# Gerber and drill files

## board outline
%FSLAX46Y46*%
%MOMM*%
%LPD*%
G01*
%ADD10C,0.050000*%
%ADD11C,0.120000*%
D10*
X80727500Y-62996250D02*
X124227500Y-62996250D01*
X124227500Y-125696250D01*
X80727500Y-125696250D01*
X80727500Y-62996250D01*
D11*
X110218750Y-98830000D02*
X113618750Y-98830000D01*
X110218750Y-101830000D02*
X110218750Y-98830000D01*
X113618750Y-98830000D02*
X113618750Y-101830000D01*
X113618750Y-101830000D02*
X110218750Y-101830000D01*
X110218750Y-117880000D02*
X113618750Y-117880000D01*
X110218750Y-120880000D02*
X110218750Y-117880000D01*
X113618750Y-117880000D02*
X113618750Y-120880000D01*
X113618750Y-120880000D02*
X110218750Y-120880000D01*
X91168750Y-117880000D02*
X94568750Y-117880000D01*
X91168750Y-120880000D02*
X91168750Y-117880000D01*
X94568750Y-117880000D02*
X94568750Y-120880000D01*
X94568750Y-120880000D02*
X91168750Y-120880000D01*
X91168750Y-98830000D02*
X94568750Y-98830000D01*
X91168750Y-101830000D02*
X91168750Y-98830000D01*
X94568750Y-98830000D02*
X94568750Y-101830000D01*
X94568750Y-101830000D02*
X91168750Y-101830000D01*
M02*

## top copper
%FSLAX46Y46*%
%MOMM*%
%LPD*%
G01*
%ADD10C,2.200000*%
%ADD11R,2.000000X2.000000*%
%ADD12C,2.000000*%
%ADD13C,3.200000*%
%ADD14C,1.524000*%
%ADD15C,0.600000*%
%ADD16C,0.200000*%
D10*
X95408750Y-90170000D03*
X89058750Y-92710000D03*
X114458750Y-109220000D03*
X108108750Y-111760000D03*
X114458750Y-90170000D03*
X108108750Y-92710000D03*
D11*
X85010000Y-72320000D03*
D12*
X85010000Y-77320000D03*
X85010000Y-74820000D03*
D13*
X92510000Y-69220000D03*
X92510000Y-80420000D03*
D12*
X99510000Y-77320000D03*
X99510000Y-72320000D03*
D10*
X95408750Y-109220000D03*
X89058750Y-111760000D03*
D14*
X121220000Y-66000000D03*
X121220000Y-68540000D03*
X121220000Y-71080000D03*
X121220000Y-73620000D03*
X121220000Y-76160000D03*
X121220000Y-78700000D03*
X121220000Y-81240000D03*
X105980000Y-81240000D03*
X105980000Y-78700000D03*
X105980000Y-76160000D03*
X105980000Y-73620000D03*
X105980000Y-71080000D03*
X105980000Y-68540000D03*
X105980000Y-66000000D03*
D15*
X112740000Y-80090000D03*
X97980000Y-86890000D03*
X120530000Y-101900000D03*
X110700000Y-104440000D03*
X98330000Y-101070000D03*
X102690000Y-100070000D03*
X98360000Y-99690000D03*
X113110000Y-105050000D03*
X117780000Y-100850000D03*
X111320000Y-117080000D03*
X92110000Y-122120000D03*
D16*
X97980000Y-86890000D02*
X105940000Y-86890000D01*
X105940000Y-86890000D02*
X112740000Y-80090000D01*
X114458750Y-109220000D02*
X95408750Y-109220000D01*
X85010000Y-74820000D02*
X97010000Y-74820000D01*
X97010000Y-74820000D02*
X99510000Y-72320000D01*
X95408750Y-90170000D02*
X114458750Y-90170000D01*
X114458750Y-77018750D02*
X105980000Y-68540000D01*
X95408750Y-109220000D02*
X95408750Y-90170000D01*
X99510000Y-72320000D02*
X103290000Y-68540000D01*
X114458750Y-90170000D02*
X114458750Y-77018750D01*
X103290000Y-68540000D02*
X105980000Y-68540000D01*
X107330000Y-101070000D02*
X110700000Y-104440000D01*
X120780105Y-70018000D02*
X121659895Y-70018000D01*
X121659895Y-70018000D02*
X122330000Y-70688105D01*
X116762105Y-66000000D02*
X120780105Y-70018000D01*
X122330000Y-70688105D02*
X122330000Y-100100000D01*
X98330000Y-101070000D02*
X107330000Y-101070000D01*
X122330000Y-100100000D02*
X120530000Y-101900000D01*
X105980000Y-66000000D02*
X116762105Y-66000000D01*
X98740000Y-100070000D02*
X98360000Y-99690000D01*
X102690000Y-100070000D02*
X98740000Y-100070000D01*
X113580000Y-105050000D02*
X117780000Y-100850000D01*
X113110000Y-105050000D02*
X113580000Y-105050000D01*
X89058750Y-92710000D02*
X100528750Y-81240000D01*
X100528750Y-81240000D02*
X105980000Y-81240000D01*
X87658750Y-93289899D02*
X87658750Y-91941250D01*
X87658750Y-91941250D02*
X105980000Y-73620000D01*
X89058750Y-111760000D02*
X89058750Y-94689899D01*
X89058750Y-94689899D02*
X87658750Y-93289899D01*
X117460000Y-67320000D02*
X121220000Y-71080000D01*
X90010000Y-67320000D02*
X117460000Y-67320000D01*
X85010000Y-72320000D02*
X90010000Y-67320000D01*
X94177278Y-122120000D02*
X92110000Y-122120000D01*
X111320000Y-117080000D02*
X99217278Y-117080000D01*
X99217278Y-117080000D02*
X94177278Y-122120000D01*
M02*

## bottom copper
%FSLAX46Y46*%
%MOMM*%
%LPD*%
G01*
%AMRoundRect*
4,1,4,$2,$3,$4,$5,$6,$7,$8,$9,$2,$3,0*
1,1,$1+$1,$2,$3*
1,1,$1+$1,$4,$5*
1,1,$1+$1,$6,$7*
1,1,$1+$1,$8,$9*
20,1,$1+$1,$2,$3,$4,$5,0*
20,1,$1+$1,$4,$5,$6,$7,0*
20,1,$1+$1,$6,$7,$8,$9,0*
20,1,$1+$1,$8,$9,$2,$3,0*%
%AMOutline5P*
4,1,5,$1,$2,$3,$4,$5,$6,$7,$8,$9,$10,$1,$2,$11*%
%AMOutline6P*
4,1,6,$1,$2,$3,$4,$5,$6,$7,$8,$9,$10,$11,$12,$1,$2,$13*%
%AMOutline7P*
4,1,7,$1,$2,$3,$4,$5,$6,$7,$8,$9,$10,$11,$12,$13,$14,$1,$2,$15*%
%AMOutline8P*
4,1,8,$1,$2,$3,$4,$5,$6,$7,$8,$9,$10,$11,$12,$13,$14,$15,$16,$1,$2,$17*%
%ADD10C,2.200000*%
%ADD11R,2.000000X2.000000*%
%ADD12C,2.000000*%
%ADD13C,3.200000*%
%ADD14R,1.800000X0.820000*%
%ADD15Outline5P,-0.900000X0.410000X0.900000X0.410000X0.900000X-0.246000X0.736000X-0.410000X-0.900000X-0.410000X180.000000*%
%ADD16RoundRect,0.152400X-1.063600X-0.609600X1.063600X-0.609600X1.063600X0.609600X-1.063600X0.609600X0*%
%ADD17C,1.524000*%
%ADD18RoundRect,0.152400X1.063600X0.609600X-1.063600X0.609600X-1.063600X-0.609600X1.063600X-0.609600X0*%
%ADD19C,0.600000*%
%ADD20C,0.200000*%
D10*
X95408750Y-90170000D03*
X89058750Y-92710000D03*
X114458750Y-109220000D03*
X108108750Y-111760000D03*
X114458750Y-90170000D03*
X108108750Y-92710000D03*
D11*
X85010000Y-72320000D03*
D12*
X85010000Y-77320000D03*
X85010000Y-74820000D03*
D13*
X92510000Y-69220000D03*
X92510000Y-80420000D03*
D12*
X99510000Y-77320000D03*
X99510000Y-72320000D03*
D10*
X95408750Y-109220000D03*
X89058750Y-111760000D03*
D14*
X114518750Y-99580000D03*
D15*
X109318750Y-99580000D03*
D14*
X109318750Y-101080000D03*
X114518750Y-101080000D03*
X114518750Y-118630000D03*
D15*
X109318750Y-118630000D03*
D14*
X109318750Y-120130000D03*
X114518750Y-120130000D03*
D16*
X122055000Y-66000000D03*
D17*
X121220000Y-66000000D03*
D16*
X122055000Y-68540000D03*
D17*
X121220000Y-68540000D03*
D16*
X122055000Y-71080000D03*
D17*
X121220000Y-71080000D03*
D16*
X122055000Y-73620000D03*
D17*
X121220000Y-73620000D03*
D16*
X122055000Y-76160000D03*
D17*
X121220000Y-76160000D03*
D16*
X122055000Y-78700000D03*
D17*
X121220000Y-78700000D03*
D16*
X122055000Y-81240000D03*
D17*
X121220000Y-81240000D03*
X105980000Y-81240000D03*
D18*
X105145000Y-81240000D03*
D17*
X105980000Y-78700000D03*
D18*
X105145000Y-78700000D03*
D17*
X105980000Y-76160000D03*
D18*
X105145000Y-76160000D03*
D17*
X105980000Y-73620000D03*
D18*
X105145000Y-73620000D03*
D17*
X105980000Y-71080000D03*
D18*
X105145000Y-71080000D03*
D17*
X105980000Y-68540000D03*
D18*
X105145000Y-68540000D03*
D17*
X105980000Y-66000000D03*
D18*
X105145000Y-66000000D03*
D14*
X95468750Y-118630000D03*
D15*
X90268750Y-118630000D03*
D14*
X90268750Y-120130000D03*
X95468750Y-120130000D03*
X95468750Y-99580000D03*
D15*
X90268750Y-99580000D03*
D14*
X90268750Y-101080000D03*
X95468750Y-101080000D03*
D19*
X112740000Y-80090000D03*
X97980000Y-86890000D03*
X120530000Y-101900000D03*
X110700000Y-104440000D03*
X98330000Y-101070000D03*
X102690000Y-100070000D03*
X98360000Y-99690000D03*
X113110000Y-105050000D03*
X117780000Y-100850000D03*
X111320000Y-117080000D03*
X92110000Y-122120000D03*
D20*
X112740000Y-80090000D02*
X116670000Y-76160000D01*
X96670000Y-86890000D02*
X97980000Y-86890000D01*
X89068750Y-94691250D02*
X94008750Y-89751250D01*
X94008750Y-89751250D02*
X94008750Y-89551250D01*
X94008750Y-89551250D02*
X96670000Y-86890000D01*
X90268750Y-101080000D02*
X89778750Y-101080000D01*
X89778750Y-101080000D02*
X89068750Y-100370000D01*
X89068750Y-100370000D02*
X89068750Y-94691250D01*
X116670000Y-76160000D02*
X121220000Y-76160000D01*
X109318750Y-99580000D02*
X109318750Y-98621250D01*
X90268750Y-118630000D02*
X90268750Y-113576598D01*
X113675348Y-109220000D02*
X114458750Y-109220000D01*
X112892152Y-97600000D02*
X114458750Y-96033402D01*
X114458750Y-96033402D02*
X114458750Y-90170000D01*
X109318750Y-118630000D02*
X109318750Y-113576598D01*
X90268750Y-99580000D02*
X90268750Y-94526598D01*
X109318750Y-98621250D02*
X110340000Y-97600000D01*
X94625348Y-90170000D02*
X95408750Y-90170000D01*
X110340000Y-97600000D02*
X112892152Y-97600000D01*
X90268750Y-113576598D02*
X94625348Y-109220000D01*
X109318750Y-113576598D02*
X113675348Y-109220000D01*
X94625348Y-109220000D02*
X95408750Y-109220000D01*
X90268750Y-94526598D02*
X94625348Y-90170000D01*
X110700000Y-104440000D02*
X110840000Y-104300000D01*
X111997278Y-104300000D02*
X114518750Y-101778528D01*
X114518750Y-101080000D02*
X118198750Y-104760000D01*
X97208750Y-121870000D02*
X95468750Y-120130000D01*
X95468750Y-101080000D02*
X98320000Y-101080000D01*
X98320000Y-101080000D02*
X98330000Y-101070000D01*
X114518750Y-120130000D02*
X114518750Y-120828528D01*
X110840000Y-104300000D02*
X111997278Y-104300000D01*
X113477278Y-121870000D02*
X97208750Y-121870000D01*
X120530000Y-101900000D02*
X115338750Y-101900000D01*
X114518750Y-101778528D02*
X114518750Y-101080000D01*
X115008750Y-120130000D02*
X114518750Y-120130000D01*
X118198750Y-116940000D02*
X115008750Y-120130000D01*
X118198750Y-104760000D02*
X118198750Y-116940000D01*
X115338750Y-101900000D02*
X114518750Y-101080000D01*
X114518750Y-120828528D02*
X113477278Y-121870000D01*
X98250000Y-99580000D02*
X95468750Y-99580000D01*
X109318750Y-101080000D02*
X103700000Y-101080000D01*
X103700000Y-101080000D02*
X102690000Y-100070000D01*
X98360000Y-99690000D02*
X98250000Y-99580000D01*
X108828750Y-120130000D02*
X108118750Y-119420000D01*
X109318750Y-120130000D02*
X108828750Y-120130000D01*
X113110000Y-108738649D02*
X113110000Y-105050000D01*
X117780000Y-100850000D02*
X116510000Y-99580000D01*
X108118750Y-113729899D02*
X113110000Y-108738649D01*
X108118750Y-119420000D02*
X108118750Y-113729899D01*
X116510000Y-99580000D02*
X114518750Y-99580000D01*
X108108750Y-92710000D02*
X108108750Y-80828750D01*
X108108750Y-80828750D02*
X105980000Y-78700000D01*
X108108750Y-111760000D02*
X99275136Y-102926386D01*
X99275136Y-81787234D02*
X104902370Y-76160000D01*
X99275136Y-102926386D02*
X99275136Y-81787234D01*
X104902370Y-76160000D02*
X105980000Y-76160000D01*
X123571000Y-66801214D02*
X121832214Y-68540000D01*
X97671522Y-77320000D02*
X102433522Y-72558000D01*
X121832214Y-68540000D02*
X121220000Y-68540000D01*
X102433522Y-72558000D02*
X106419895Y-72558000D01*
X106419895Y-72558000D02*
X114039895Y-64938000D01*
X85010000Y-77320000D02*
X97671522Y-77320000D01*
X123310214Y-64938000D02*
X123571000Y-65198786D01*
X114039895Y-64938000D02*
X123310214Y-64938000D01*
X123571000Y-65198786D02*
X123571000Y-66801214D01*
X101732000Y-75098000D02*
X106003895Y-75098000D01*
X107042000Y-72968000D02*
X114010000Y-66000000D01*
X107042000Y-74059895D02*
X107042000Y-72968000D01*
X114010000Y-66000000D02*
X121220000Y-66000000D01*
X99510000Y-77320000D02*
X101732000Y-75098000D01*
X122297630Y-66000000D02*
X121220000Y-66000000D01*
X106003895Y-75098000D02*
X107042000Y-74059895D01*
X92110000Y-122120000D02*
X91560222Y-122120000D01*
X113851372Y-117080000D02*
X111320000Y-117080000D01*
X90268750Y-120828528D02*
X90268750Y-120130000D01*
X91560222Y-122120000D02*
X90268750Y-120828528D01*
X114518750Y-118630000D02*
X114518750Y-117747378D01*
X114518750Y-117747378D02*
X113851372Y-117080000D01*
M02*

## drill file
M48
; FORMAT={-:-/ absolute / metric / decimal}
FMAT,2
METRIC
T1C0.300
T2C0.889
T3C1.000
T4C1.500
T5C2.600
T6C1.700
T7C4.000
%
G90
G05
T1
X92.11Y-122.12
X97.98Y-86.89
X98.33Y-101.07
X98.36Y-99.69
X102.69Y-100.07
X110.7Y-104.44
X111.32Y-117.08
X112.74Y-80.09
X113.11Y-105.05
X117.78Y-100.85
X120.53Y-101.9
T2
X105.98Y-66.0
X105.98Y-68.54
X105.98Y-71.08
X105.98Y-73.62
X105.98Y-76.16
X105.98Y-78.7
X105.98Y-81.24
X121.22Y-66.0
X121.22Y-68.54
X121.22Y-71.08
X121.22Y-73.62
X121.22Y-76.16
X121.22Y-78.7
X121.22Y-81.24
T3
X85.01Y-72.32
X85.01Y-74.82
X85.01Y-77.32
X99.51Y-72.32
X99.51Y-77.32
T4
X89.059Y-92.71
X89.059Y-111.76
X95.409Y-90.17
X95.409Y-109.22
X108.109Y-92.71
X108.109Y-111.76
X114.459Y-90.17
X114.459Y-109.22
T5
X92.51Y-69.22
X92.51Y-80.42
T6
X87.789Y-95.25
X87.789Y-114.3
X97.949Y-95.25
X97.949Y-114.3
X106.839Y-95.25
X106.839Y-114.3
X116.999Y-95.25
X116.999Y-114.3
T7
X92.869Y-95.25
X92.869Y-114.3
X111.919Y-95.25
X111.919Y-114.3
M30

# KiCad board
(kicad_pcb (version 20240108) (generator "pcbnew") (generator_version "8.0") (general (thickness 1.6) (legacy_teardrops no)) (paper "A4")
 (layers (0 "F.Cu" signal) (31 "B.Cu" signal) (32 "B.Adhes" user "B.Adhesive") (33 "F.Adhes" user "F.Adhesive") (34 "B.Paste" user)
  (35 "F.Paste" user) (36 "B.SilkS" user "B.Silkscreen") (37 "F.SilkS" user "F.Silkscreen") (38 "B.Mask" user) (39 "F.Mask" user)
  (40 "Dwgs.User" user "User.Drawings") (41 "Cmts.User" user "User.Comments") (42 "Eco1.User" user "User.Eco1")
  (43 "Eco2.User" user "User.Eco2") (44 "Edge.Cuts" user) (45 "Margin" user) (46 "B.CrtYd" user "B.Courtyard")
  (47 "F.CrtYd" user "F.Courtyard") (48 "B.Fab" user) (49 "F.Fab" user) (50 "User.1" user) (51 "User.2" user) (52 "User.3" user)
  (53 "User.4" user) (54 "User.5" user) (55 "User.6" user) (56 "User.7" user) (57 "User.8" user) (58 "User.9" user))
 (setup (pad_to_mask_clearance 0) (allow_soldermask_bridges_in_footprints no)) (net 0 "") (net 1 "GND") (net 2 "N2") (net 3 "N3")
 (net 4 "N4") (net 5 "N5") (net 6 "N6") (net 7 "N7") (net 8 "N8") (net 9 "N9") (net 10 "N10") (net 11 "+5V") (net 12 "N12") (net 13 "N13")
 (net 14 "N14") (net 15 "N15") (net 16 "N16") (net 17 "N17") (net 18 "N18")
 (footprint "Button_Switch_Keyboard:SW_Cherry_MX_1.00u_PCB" (layer "F.Cu") (at 95.40875 90.17)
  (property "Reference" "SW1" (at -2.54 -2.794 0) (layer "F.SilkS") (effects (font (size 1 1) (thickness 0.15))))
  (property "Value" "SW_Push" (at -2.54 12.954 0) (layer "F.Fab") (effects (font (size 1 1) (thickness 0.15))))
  (pad "" np_thru_hole circle (at -7.62 5.08) (size 1.7 1.7) (drill 1.7) (layers "*.Cu" "*.Mask"))
  (pad "" np_thru_hole circle (at -2.54 5.08) (size 4 4) (drill 4) (layers "*.Cu" "*.Mask"))
  (pad "" np_thru_hole circle (at 2.54 5.08) (size 1.7 1.7) (drill 1.7) (layers "*.Cu" "*.Mask"))
  (pad "1" thru_hole circle (at 0 0) (size 2.2 2.2) (drill 1.5) (layers "*.Cu" "*.Mask") (remove_unused_layers no) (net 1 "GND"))
  (pad "2" thru_hole circle (at -6.35 2.54) (size 2.2 2.2) (drill 1.5) (layers "*.Cu" "*.Mask") (remove_unused_layers no) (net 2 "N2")))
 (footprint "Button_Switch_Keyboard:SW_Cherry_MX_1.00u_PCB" (layer "F.Cu") (at 114.45875 109.22)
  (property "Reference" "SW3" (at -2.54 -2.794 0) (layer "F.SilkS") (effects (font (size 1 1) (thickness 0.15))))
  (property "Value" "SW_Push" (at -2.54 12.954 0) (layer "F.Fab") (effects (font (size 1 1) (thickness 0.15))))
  (pad "" np_thru_hole circle (at -7.62 5.08) (size 1.7 1.7) (drill 1.7) (layers "*.Cu" "*.Mask"))
  (pad "" np_thru_hole circle (at -2.54 5.08) (size 4 4) (drill 4) (layers "*.Cu" "*.Mask"))
  (pad "" np_thru_hole circle (at 2.54 5.08) (size 1.7 1.7) (drill 1.7) (layers "*.Cu" "*.Mask"))
  (pad "1" thru_hole circle (at 0 0) (size 2.2 2.2) (drill 1.5) (layers "*.Cu" "*.Mask") (remove_unused_layers no) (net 1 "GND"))
  (pad "2" thru_hole circle (at -6.35 2.54) (size 2.2 2.2) (drill 1.5) (layers "*.Cu" "*.Mask") (remove_unused_layers no) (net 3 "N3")))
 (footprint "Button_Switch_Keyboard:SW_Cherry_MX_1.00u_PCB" (layer "F.Cu") (at 114.45875 90.17)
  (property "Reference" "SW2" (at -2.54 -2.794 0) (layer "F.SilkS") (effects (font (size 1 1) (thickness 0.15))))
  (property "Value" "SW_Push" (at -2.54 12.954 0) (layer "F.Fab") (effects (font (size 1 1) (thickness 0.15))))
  (pad "" np_thru_hole circle (at -7.62 5.08) (size 1.7 1.7) (drill 1.7) (layers "*.Cu" "*.Mask"))
  (pad "" np_thru_hole circle (at -2.54 5.08) (size 4 4) (drill 4) (layers "*.Cu" "*.Mask"))
  (pad "" np_thru_hole circle (at 2.54 5.08) (size 1.7 1.7) (drill 1.7) (layers "*.Cu" "*.Mask"))
  (pad "1" thru_hole circle (at 0 0) (size 2.2 2.2) (drill 1.5) (layers "*.Cu" "*.Mask") (remove_unused_layers no) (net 1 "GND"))
  (pad "2" thru_hole circle (at -6.35 2.54) (size 2.2 2.2) (drill 1.5) (layers "*.Cu" "*.Mask") (remove_unused_layers no) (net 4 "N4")))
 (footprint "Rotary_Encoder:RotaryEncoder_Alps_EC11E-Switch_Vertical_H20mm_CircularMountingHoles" (layer "F.Cu") (at 85.01 72.32)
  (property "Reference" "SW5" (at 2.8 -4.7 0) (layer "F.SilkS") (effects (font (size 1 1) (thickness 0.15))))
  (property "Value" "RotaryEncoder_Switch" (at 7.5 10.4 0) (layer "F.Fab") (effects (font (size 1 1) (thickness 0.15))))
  (pad "A" thru_hole rect (at 0 0) (size 2 2) (drill 1) (layers "*.Cu" "*.Mask") (remove_unused_layers no) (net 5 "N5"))
  (pad "B" thru_hole circle (at 0 5) (size 2 2) (drill 1) (layers "*.Cu" "*.Mask") (remove_unused_layers no) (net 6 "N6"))
  (pad "C" thru_hole circle (at 0 2.5) (size 2 2) (drill 1) (layers "*.Cu" "*.Mask") (remove_unused_layers no) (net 1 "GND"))
  (pad "MP" thru_hole circle (at 7.5 -3.1) (size 3.2 3.2) (drill 2.6) (layers "*.Cu" "*.Mask") (remove_unused_layers no))
  (pad "MP" thru_hole circle (at 7.5 8.1) (size 3.2 3.2) (drill 2.6) (layers "*.Cu" "*.Mask") (remove_unused_layers no))
  (pad "S1" thru_hole circle (at 14.5 5) (size 2 2) (drill 1) (layers "*.Cu" "*.Mask") (remove_unused_layers no) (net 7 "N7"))
  (pad "S2" thru_hole circle (at 14.5 0) (size 2 2) (drill 1) (layers "*.Cu" "*.Mask") (remove_unused_layers no) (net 1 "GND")))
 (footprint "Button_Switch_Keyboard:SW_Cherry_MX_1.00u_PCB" (layer "F.Cu") (at 95.40875 109.22)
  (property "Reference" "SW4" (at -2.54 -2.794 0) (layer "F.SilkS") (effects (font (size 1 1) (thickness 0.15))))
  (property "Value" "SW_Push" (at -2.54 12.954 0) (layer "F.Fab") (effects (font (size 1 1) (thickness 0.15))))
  (pad "" np_thru_hole circle (at -7.62 5.08) (size 1.7 1.7) (drill 1.7) (layers "*.Cu" "*.Mask"))
  (pad "" np_thru_hole circle (at -2.54 5.08) (size 4 4) (drill 4) (layers "*.Cu" "*.Mask"))
  (pad "" np_thru_hole circle (at 2.54 5.08) (size 1.7 1.7) (drill 1.7) (layers "*.Cu" "*.Mask"))
  (pad "1" thru_hole circle (at 0 0) (size 2.2 2.2) (drill 1.5) (layers "*.Cu" "*.Mask") (remove_unused_layers no) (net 1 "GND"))
  (pad "2" thru_hole circle (at -6.35 2.54) (size 2.2 2.2) (drill 1.5) (layers "*.Cu" "*.Mask") (remove_unused_layers no) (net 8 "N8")))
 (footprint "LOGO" (layer "B.Cu") (at 101.67 98.78 180)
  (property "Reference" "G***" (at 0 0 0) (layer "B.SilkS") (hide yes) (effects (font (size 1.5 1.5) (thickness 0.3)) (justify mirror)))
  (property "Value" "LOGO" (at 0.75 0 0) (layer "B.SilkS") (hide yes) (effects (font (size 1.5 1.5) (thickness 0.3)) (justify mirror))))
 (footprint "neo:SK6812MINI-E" (layer "B.Cu") (at 111.91875 100.33 180)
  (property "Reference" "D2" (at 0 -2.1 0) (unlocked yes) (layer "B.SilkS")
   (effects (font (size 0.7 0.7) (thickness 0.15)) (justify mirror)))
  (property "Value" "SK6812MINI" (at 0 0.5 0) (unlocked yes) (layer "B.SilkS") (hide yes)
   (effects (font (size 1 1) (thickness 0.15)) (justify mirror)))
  (fp_line (start 1.7 1.5) (end -1.7 1.5) (stroke (width 0.12) (type solid)) (layer "Edge.Cuts"))
  (fp_line (start 1.7 -1.5) (end 1.7 1.5) (stroke (width 0.12) (type solid)) (layer "Edge.Cuts"))
  (fp_line (start -1.7 1.5) (end -1.7 -1.5) (stroke (width 0.12) (type solid)) (layer "Edge.Cuts"))
  (fp_line (start -1.7 -1.5) (end 1.7 -1.5) (stroke (width 0.12) (type solid)) (layer "Edge.Cuts"))
  (pad "1" smd rect (at -2.6 0.75 180) (size 1.8 0.82) (layers "B.Cu" "B.Paste" "B.Mask") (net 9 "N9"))
  (pad "2" smd roundrect (at 2.6 0.75 180) (size 1.8 0.82) (layers "B.Cu" "B.Paste" "B.Mask") (roundrect_rratio 0) (chamfer_ratio 0.2)
   (chamfer bottom_right) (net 1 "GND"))
  (pad "3" smd rect (at 2.6 -0.75 180) (size 1.8 0.82) (layers "B.Cu" "B.Paste" "B.Mask") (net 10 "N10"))
  (pad "4" smd rect (at -2.6 -0.75 180) (size 1.8 0.82) (layers "B.Cu" "B.Paste" "B.Mask") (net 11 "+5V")))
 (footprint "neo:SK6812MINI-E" (layer "B.Cu") (at 111.91875 119.38 180)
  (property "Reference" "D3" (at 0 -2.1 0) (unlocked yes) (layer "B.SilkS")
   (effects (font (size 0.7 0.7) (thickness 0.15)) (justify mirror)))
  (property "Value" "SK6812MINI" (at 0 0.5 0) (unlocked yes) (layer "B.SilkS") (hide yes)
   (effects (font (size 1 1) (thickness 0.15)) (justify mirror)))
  (fp_line (start 1.7 1.5) (end -1.7 1.5) (stroke (width 0.12) (type solid)) (layer "Edge.Cuts"))
  (fp_line (start 1.7 -1.5) (end 1.7 1.5) (stroke (width 0.12) (type solid)) (layer "Edge.Cuts"))
  (fp_line (start -1.7 1.5) (end -1.7 -1.5) (stroke (width 0.12) (type solid)) (layer "Edge.Cuts"))
  (fp_line (start -1.7 -1.5) (end 1.7 -1.5) (stroke (width 0.12) (type solid)) (layer "Edge.Cuts"))
  (pad "1" smd rect (at -2.6 0.75 180) (size 1.8 0.82) (layers "B.Cu" "B.Paste" "B.Mask") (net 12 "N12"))
  (pad "2" smd roundrect (at 2.6 0.75 180) (size 1.8 0.82) (layers "B.Cu" "B.Paste" "B.Mask") (roundrect_rratio 0) (chamfer_ratio 0.2)
   (chamfer bottom_right) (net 1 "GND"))
  (pad "3" smd rect (at 2.6 -0.75 180) (size 1.8 0.82) (layers "B.Cu" "B.Paste" "B.Mask") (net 9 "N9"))
  (pad "4" smd rect (at -2.6 -0.75 180) (size 1.8 0.82) (layers "B.Cu" "B.Paste" "B.Mask") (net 11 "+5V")))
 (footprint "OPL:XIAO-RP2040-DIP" (layer "B.Cu") (at 113.6 73.62 180)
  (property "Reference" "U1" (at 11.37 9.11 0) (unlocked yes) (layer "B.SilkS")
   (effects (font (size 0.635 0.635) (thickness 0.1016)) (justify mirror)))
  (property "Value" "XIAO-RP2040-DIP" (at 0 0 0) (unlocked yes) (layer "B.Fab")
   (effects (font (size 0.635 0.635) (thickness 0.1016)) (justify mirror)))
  (pad "1" smd roundrect (at -8.455 7.62) (size 2.432 1.524) (layers "B.Cu" "B.Mask") (roundrect_rratio 0.1) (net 7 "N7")
   (thermal_bridge_angle 45))
  (pad "1" thru_hole circle (at -7.62 7.62) (size 1.524 1.524) (drill 0.889) (layers "*.Cu" "*.Mask") (remove_unused_layers no) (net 7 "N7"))
  (pad "2" smd roundrect (at -8.455 5.08) (size 2.432 1.524) (layers "B.Cu" "B.Mask") (roundrect_rratio 0.1) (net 6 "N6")
   (thermal_bridge_angle 45))
  (pad "2" thru_hole circle (at -7.62 5.08) (size 1.524 1.524) (drill 0.889) (layers "*.Cu" "*.Mask") (remove_unused_layers no) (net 6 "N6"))
  (pad "3" smd roundrect (at -8.455 2.54) (size 2.432 1.524) (layers "B.Cu" "B.Mask") (roundrect_rratio 0.1) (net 5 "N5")
   (thermal_bridge_angle 45))
  (pad "3" thru_hole circle (at -7.62 2.54) (size 1.524 1.524) (drill 0.889) (layers "*.Cu" "*.Mask") (remove_unused_layers no) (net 5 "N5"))
  (pad "4" smd roundrect (at -8.455 0) (size 2.432 1.524) (layers "B.Cu" "B.Mask") (roundrect_rratio 0.1) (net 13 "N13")
   (thermal_bridge_angle 45))
  (pad "4" thru_hole circle (at -7.62 0) (size 1.524 1.524) (drill 0.889) (layers "*.Cu" "*.Mask") (remove_unused_layers no) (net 13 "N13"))
  (pad "5" smd roundrect (at -8.455 -2.54) (size 2.432 1.524) (layers "B.Cu" "B.Mask") (roundrect_rratio 0.1) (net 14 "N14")
   (thermal_bridge_angle 45))
  (pad "5" thru_hole circle (at -7.62 -2.54) (size 1.524 1.524) (drill 0.889) (layers "*.Cu" "*.Mask") (remove_unused_layers no)
   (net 14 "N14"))
  (pad "6" smd roundrect (at -8.455 -5.08) (size 2.432 1.524) (layers "B.Cu" "B.Mask") (roundrect_rratio 0.1) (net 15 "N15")
   (thermal_bridge_angle 45))
  (pad "6" thru_hole circle (at -7.62 -5.08) (size 1.524 1.524) (drill 0.889) (layers "*.Cu" "*.Mask") (remove_unused_layers no)
   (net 15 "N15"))
  (pad "7" smd roundrect (at -8.455 -7.62) (size 2.432 1.524) (layers "B.Cu" "B.Mask") (roundrect_rratio 0.1) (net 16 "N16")
   (thermal_bridge_angle 45))
  (pad "7" thru_hole circle (at -7.62 -7.62) (size 1.524 1.524) (drill 0.889) (layers "*.Cu" "*.Mask") (remove_unused_layers no)
   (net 16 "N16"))
  (pad "8" thru_hole circle (at 7.62 -7.62 180) (size 1.524 1.524) (drill 0.889) (layers "*.Cu" "*.Mask") (remove_unused_layers no)
   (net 2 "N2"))
  (pad "8" smd roundrect (at 8.455 -7.62 180) (size 2.432 1.524) (layers "B.Cu" "B.Mask") (roundrect_rratio 0.1) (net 2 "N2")
   (thermal_bridge_angle 45))
  (pad "9" thru_hole circle (at 7.62 -5.08 180) (size 1.524 1.524) (drill 0.889) (layers "*.Cu" "*.Mask") (remove_unused_layers no)
   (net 4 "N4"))
  (pad "9" smd roundrect (at 8.455 -5.08 180) (size 2.432 1.524) (layers "B.Cu" "B.Mask") (roundrect_rratio 0.1) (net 4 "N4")
   (thermal_bridge_angle 45))
  (pad "10" thru_hole circle (at 7.62 -2.54 180) (size 1.524 1.524) (drill 0.889) (layers "*.Cu" "*.Mask") (remove_unused_layers no)
   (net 3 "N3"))
  (pad "10" smd roundrect (at 8.455 -2.54 180) (size 2.432 1.524) (layers "B.Cu" "B.Mask") (roundrect_rratio 0.1) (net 3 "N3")
   (thermal_bridge_angle 45))
  (pad "11" thru_hole circle (at 7.62 0 180) (size 1.524 1.524) (drill 0.889) (layers "*.Cu" "*.Mask") (remove_unused_layers no)
   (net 8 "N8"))
  (pad "11" smd roundrect (at 8.455 0 180) (size 2.432 1.524) (layers "B.Cu" "B.Mask") (roundrect_rratio 0.1) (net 8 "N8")
   (thermal_bridge_angle 45))
  (pad "12" thru_hole circle (at 7.62 2.54 180) (size 1.524 1.524) (drill 0.889) (layers "*.Cu" "*.Mask") (remove_unused_layers no)
   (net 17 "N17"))
  (pad "12" smd roundrect (at 8.455 2.54 180) (size 2.432 1.524) (layers "B.Cu" "B.Mask") (roundrect_rratio 0.1) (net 17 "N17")
   (thermal_bridge_angle 45))
  (pad "13" thru_hole circle (at 7.62 5.08 180) (size 1.524 1.524) (drill 0.889) (layers "*.Cu" "*.Mask") (remove_unused_layers no)
   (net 1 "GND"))
  (pad "13" smd roundrect (at 8.455 5.08 180) (size 2.432 1.524) (layers "B.Cu" "B.Mask") (roundrect_rratio 0.1) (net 1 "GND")
   (thermal_bridge_angle 45))
  (pad "14" thru_hole circle (at 7.62 7.62 180) (size 1.524 1.524) (drill 0.889) (layers "*.Cu" "*.Mask") (remove_unused_layers no)
   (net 11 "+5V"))
  (pad "14" smd roundrect (at 8.455 7.62 180) (size 2.432 1.524) (layers "B.Cu" "B.Mask") (roundrect_rratio 0.1) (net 11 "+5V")
   (thermal_bridge_angle 45)))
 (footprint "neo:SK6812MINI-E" (layer "B.Cu") (at 92.86875 119.38 180)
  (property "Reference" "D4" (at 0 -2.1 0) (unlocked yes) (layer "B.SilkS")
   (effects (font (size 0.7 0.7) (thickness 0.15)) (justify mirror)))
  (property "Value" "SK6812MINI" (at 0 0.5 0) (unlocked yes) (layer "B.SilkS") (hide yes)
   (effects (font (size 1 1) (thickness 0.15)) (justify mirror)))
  (fp_line (start 1.7 1.5) (end -1.7 1.5) (stroke (width 0.12) (type solid)) (layer "Edge.Cuts"))
  (fp_line (start 1.7 -1.5) (end 1.7 1.5) (stroke (width 0.12) (type solid)) (layer "Edge.Cuts"))
  (fp_line (start -1.7 1.5) (end -1.7 -1.5) (stroke (width 0.12) (type solid)) (layer "Edge.Cuts"))
  (fp_line (start -1.7 -1.5) (end 1.7 -1.5) (stroke (width 0.12) (type solid)) (layer "Edge.Cuts"))
  (pad "1" smd rect (at -2.6 0.75 180) (size 1.8 0.82) (layers "B.Cu" "B.Paste" "B.Mask") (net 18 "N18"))
  (pad "2" smd roundrect (at 2.6 0.75 180) (size 1.8 0.82) (layers "B.Cu" "B.Paste" "B.Mask") (roundrect_rratio 0) (chamfer_ratio 0.2)
   (chamfer bottom_right) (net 1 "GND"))
  (pad "3" smd rect (at 2.6 -0.75 180) (size 1.8 0.82) (layers "B.Cu" "B.Paste" "B.Mask") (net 12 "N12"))
  (pad "4" smd rect (at -2.6 -0.75 180) (size 1.8 0.82) (layers "B.Cu" "B.Paste" "B.Mask") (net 11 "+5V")))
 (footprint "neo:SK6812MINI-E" (layer "B.Cu") (at 92.86875 100.33 180)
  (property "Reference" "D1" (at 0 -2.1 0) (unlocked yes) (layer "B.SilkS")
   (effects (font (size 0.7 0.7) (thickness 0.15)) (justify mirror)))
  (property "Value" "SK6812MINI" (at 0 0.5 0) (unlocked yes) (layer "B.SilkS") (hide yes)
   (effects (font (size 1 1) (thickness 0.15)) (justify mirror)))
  (fp_line (start 1.7 1.5) (end -1.7 1.5) (stroke (width 0.12) (type solid)) (layer "Edge.Cuts"))
  (fp_line (start 1.7 -1.5) (end 1.7 1.5) (stroke (width 0.12) (type solid)) (layer "Edge.Cuts"))
  (fp_line (start -1.7 1.5) (end -1.7 -1.5) (stroke (width 0.12) (type solid)) (layer "Edge.Cuts"))
  (fp_line (start -1.7 -1.5) (end 1.7 -1.5) (stroke (width 0.12) (type solid)) (layer "Edge.Cuts"))
  (pad "1" smd rect (at -2.6 0.75 180) (size 1.8 0.82) (layers "B.Cu" "B.Paste" "B.Mask") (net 10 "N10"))
  (pad "2" smd roundrect (at 2.6 0.75 180) (size 1.8 0.82) (layers "B.Cu" "B.Paste" "B.Mask") (roundrect_rratio 0) (chamfer_ratio 0.2)
   (chamfer bottom_right) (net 1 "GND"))
  (pad "3" smd rect (at 2.6 -0.75 180) (size 1.8 0.82) (layers "B.Cu" "B.Paste" "B.Mask") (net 14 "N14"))
  (pad "4" smd rect (at -2.6 -0.75 180) (size 1.8 0.82) (layers "B.Cu" "B.Paste" "B.Mask") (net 11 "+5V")))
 (gr_rect (start 80.7275 62.99625) (end 124.2275 125.69625) (stroke (width 0.05) (type default)) (fill none) (layer "Edge.Cuts"))
 (segment (start 97.98 86.89) (end 105.94 86.89) (width 0.2) (layer "F.Cu") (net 14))
 (segment (start 105.94 86.89) (end 112.74 80.09) (width 0.2) (layer "F.Cu") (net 14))
 (via (at 112.74 80.09) (size 0.6) (drill 0.3) (layers "F.Cu" "B.Cu") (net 14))
 (via (at 97.98 86.89) (size 0.6) (drill 0.3) (layers "F.Cu" "B.Cu") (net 14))
 (segment (start 112.74 80.09) (end 116.67 76.16) (width 0.2) (layer "B.Cu") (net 14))
 (segment (start 96.67 86.89) (end 97.98 86.89) (width 0.2) (layer "B.Cu") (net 14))
 (segment (start 89.06875 94.69125) (end 94.00875 89.75125) (width 0.2) (layer "B.Cu") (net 14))
 (segment (start 94.00875 89.75125) (end 94.00875 89.55125) (width 0.2) (layer "B.Cu") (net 14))
 (segment (start 94.00875 89.55125) (end 96.67 86.89) (width 0.2) (layer "B.Cu") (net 14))
 (segment (start 90.26875 101.08) (end 89.77875 101.08) (width 0.2) (layer "B.Cu") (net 14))
 (segment (start 89.77875 101.08) (end 89.06875 100.37) (width 0.2) (layer "B.Cu") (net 14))
 (segment (start 89.06875 100.37) (end 89.06875 94.69125) (width 0.2) (layer "B.Cu") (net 14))
 (segment (start 116.67 76.16) (end 121.22 76.16) (width 0.2) (layer "B.Cu") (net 14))
 (segment (start 114.45875 109.22) (end 95.40875 109.22) (width 0.2) (layer "F.Cu") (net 1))
 (segment (start 85.01 74.82) (end 97.01 74.82) (width 0.2) (layer "F.Cu") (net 1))
 (segment (start 97.01 74.82) (end 99.51 72.32) (width 0.2) (layer "F.Cu") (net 1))
 (segment (start 95.40875 90.17) (end 114.45875 90.17) (width 0.2) (layer "F.Cu") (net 1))
 (segment (start 114.45875 77.01875) (end 105.98 68.54) (width 0.2) (layer "F.Cu") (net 1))
 (segment (start 95.40875 109.22) (end 95.40875 90.17) (width 0.2) (layer "F.Cu") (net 1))
 (segment (start 99.51 72.32) (end 103.29 68.54) (width 0.2) (layer "F.Cu") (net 1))
 (segment (start 114.45875 90.17) (end 114.45875 77.01875) (width 0.2) (layer "F.Cu") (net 1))
 (segment (start 103.29 68.54) (end 105.98 68.54) (width 0.2) (layer "F.Cu") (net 1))
 (segment (start 109.31875 99.58) (end 109.31875 98.62125) (width 0.2) (layer "B.Cu") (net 1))
 (segment (start 90.26875 118.63) (end 90.26875 113.576598) (width 0.2) (layer "B.Cu") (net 1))
 (segment (start 113.675348 109.22) (end 114.45875 109.22) (width 0.2) (layer "B.Cu") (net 1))
 (segment (start 112.892152 97.6) (end 114.45875 96.033402) (width 0.2) (layer "B.Cu") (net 1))
 (segment (start 114.45875 96.033402) (end 114.45875 90.17) (width 0.2) (layer "B.Cu") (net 1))
 (segment (start 109.31875 118.63) (end 109.31875 113.576598) (width 0.2) (layer "B.Cu") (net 1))
 (segment (start 90.26875 99.58) (end 90.26875 94.526598) (width 0.2) (layer "B.Cu") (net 1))
 (segment (start 109.31875 98.62125) (end 110.34 97.6) (width 0.2) (layer "B.Cu") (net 1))
 (segment (start 94.625348 90.17) (end 95.40875 90.17) (width 0.2) (layer "B.Cu") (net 1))
 (segment (start 110.34 97.6) (end 112.892152 97.6) (width 0.2) (layer "B.Cu") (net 1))
 (segment (start 90.26875 113.576598) (end 94.625348 109.22) (width 0.2) (layer "B.Cu") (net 1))
 (segment (start 109.31875 113.576598) (end 113.675348 109.22) (width 0.2) (layer "B.Cu") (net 1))
 (segment (start 94.625348 109.22) (end 95.40875 109.22) (width 0.2) (layer "B.Cu") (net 1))
 (segment (start 90.26875 94.526598) (end 94.625348 90.17) (width 0.2) (layer "B.Cu") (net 1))
 (segment (start 107.33 101.07) (end 110.7 104.44) (width 0.2) (layer "F.Cu") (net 11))
 (segment (start 120.780105 70.018) (end 121.659895 70.018) (width 0.2) (layer "F.Cu") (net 11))
 (segment (start 121.659895 70.018) (end 122.33 70.688105) (width 0.2) (layer "F.Cu") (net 11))
 (segment (start 116.762105 66) (end 120.780105 70.018) (width 0.2) (layer "F.Cu") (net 11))
 (segment (start 122.33 70.688105) (end 122.33 100.1) (width 0.2) (layer "F.Cu") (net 11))
 (segment (start 98.33 101.07) (end 107.33 101.07) (width 0.2) (layer "F.Cu") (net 11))
 (segment (start 122.33 100.1) (end 120.53 101.9) (width 0.2) (layer "F.Cu") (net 11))
 (segment (start 105.98 66) (end 116.762105 66) (width 0.2) (layer "F.Cu") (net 11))
 (via (at 120.53 101.9) (size 0.6) (drill 0.3) (layers "F.Cu" "B.Cu") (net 11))
 (via (at 110.7 104.44) (size 0.6) (drill 0.3) (layers "F.Cu" "B.Cu") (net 11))
 (via (at 98.33 101.07) (size 0.6) (drill 0.3) (layers "F.Cu" "B.Cu") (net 11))
 (segment (start 110.7 104.44) (end 110.84 104.3) (width 0.2) (layer "B.Cu") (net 11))
 (segment (start 111.997278 104.3) (end 114.51875 101.778528) (width 0.2) (layer "B.Cu") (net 11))
 (segment (start 114.51875 101.08) (end 118.19875 104.76) (width 0.2) (layer "B.Cu") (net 11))
 (segment (start 97.20875 121.87) (end 95.46875 120.13) (width 0.2) (layer "B.Cu") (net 11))
 (segment (start 95.46875 101.08) (end 98.32 101.08) (width 0.2) (layer "B.Cu") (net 11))
 (segment (start 98.32 101.08) (end 98.33 101.07) (width 0.2) (layer "B.Cu") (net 11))
 (segment (start 114.51875 120.13) (end 114.51875 120.828528) (width 0.2) (layer "B.Cu") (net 11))
 (segment (start 110.84 104.3) (end 111.997278 104.3) (width 0.2) (layer "B.Cu") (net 11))
 (segment (start 113.477278 121.87) (end 97.20875 121.87) (width 0.2) (layer "B.Cu") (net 11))
 (segment (start 120.53 101.9) (end 115.33875 101.9) (width 0.2) (layer "B.Cu") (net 11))
 (segment (start 114.51875 101.778528) (end 114.51875 101.08) (width 0.2) (layer "B.Cu") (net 11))
 (segment (start 115.00875 120.13) (end 114.51875 120.13) (width 0.2) (layer "B.Cu") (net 11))
 (segment (start 118.19875 116.94) (end 115.00875 120.13) (width 0.2) (layer "B.Cu") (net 11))
 (segment (start 118.19875 104.76) (end 118.19875 116.94) (width 0.2) (layer "B.Cu") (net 11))
 (segment (start 115.33875 101.9) (end 114.51875 101.08) (width 0.2) (layer "B.Cu") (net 11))
 (segment (start 114.51875 120.828528) (end 113.477278 121.87) (width 0.2) (layer "B.Cu") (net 11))
 (segment (start 98.74 100.07) (end 98.36 99.69) (width 0.2) (layer "F.Cu") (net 10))
 (segment (start 102.69 100.07) (end 98.74 100.07) (width 0.2) (layer "F.Cu") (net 10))
 (via (at 102.69 100.07) (size 0.6) (drill 0.3) (layers "F.Cu" "B.Cu") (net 10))
 (via (at 98.36 99.69) (size 0.6) (drill 0.3) (layers "F.Cu" "B.Cu") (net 10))
 (segment (start 98.25 99.58) (end 95.46875 99.58) (width 0.2) (layer "B.Cu") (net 10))
 (segment (start 109.31875 101.08) (end 103.7 101.08) (width 0.2) (layer "B.Cu") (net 10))
 (segment (start 103.7 101.08) (end 102.69 100.07) (width 0.2) (layer "B.Cu") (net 10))
 (segment (start 98.36 99.69) (end 98.25 99.58) (width 0.2) (layer "B.Cu") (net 10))
 (segment (start 113.58 105.05) (end 117.78 100.85) (width 0.2) (layer "F.Cu") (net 9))
 (segment (start 113.11 105.05) (end 113.58 105.05) (width 0.2) (layer "F.Cu") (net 9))
 (via (at 113.11 105.05) (size 0.6) (drill 0.3) (layers "F.Cu" "B.Cu") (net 9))
 (via (at 117.78 100.85) (size 0.6) (drill 0.3) (layers "F.Cu" "B.Cu") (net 9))
 (segment (start 108.82875 120.13) (end 108.11875 119.42) (width 0.2) (layer "B.Cu") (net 9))
 (segment (start 109.31875 120.13) (end 108.82875 120.13) (width 0.2) (layer "B.Cu") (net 9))
 (segment (start 113.11 108.738649) (end 113.11 105.05) (width 0.2) (layer "B.Cu") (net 9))
 (segment (start 117.78 100.85) (end 116.51 99.58) (width 0.2) (layer "B.Cu") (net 9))
 (segment (start 108.11875 113.729899) (end 113.11 108.738649) (width 0.2) (layer "B.Cu") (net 9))
 (segment (start 108.11875 119.42) (end 108.11875 113.729899) (width 0.2) (layer "B.Cu") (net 9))
 (segment (start 116.51 99.58) (end 114.51875 99.58) (width 0.2) (layer "B.Cu") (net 9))
 (segment (start 89.05875 92.71) (end 100.52875 81.24) (width 0.2) (layer "F.Cu") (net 2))
 (segment (start 100.52875 81.24) (end 105.98 81.24) (width 0.2) (layer "F.Cu") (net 2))
 (segment (start 108.10875 92.71) (end 108.10875 80.82875) (width 0.2) (layer "B.Cu") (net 4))
 (segment (start 108.10875 80.82875) (end 105.98 78.7) (width 0.2) (layer "B.Cu") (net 4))
 (segment (start 108.10875 111.76) (end 99.275136 102.926386) (width 0.2) (layer "B.Cu") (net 3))
 (segment (start 99.275136 81.787234) (end 104.90237 76.16) (width 0.2) (layer "B.Cu") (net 3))
 (segment (start 99.275136 102.926386) (end 99.275136 81.787234) (width 0.2) (layer "B.Cu") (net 3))
 (segment (start 104.90237 76.16) (end 105.98 76.16) (width 0.2) (layer "B.Cu") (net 3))
 (segment (start 87.65875 93.289899) (end 87.65875 91.94125) (width 0.2) (layer "F.Cu") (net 8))
 (segment (start 87.65875 91.94125) (end 105.98 73.62) (width 0.2) (layer "F.Cu") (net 8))
 (segment (start 89.05875 111.76) (end 89.05875 94.689899) (width 0.2) (layer "F.Cu") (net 8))
 (segment (start 89.05875 94.689899) (end 87.65875 93.289899) (width 0.2) (layer "F.Cu") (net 8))
 (segment (start 123.571 66.801214) (end 121.832214 68.54) (width 0.2) (layer "B.Cu") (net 6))
 (segment (start 97.671522 77.32) (end 102.433522 72.558) (width 0.2) (layer "B.Cu") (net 6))
 (segment (start 121.832214 68.54) (end 121.22 68.54) (width 0.2) (layer "B.Cu") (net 6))
 (segment (start 102.433522 72.558) (end 106.419895 72.558) (width 0.2) (layer "B.Cu") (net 6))
 (segment (start 106.419895 72.558) (end 114.039895 64.938) (width 0.2) (layer "B.Cu") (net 6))
 (segment (start 85.01 77.32) (end 97.671522 77.32) (width 0.2) (layer "B.Cu") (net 6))
 (segment (start 123.310214 64.938) (end 123.571 65.198786) (width 0.2) (layer "B.Cu") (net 6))
 (segment (start 114.039895 64.938) (end 123.310214 64.938) (width 0.2) (layer "B.Cu") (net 6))
 (segment (start 123.571 65.198786) (end 123.571 66.801214) (width 0.2) (layer "B.Cu") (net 6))
 (segment (start 117.46 67.32) (end 121.22 71.08) (width 0.2) (layer "F.Cu") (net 5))
 (segment (start 90.01 67.32) (end 117.46 67.32) (width 0.2) (layer "F.Cu") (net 5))
 (segment (start 85.01 72.32) (end 90.01 67.32) (width 0.2) (layer "F.Cu") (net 5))
 (segment (start 101.732 75.098) (end 106.003895 75.098) (width 0.2) (layer "B.Cu") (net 7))
 (segment (start 107.042 72.968) (end 114.01 66) (width 0.2) (layer "B.Cu") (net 7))
 (segment (start 107.042 74.059895) (end 107.042 72.968) (width 0.2) (layer "B.Cu") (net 7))
 (segment (start 114.01 66) (end 121.22 66) (width 0.2) (layer "B.Cu") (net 7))
 (segment (start 99.51 77.32) (end 101.732 75.098) (width 0.2) (layer "B.Cu") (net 7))
 (segment (start 122.29763 66) (end 121.22 66) (width 0.2) (layer "B.Cu") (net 7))
 (segment (start 106.003895 75.098) (end 107.042 74.059895) (width 0.2) (layer "B.Cu") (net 7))
 (segment (start 94.177278 122.12) (end 92.11 122.12) (width 0.2) (layer "F.Cu") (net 12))
 (segment (start 111.32 117.08) (end 99.217278 117.08) (width 0.2) (layer "F.Cu") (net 12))
 (segment (start 99.217278 117.08) (end 94.177278 122.12) (width 0.2) (layer "F.Cu") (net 12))
 (via (at 111.32 117.08) (size 0.6) (drill 0.3) (layers "F.Cu" "B.Cu") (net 12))
 (via (at 92.11 122.12) (size 0.6) (drill 0.3) (layers "F.Cu" "B.Cu") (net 12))
 (segment (start 92.11 122.12) (end 91.560222 122.12) (width 0.2) (layer "B.Cu") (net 12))
 (segment (start 113.851372 117.08) (end 111.32 117.08) (width 0.2) (layer "B.Cu") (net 12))
 (segment (start 90.26875 120.828528) (end 90.26875 120.13) (width 0.2) (layer "B.Cu") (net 12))
 (segment (start 91.560222 122.12) (end 90.26875 120.828528) (width 0.2) (layer "B.Cu") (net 12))
 (segment (start 114.51875 118.63) (end 114.51875 117.747378) (width 0.2) (layer "B.Cu") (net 12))
 (segment (start 114.51875 117.747378) (end 113.851372 117.08) (width 0.2) (layer "B.Cu") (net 12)))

